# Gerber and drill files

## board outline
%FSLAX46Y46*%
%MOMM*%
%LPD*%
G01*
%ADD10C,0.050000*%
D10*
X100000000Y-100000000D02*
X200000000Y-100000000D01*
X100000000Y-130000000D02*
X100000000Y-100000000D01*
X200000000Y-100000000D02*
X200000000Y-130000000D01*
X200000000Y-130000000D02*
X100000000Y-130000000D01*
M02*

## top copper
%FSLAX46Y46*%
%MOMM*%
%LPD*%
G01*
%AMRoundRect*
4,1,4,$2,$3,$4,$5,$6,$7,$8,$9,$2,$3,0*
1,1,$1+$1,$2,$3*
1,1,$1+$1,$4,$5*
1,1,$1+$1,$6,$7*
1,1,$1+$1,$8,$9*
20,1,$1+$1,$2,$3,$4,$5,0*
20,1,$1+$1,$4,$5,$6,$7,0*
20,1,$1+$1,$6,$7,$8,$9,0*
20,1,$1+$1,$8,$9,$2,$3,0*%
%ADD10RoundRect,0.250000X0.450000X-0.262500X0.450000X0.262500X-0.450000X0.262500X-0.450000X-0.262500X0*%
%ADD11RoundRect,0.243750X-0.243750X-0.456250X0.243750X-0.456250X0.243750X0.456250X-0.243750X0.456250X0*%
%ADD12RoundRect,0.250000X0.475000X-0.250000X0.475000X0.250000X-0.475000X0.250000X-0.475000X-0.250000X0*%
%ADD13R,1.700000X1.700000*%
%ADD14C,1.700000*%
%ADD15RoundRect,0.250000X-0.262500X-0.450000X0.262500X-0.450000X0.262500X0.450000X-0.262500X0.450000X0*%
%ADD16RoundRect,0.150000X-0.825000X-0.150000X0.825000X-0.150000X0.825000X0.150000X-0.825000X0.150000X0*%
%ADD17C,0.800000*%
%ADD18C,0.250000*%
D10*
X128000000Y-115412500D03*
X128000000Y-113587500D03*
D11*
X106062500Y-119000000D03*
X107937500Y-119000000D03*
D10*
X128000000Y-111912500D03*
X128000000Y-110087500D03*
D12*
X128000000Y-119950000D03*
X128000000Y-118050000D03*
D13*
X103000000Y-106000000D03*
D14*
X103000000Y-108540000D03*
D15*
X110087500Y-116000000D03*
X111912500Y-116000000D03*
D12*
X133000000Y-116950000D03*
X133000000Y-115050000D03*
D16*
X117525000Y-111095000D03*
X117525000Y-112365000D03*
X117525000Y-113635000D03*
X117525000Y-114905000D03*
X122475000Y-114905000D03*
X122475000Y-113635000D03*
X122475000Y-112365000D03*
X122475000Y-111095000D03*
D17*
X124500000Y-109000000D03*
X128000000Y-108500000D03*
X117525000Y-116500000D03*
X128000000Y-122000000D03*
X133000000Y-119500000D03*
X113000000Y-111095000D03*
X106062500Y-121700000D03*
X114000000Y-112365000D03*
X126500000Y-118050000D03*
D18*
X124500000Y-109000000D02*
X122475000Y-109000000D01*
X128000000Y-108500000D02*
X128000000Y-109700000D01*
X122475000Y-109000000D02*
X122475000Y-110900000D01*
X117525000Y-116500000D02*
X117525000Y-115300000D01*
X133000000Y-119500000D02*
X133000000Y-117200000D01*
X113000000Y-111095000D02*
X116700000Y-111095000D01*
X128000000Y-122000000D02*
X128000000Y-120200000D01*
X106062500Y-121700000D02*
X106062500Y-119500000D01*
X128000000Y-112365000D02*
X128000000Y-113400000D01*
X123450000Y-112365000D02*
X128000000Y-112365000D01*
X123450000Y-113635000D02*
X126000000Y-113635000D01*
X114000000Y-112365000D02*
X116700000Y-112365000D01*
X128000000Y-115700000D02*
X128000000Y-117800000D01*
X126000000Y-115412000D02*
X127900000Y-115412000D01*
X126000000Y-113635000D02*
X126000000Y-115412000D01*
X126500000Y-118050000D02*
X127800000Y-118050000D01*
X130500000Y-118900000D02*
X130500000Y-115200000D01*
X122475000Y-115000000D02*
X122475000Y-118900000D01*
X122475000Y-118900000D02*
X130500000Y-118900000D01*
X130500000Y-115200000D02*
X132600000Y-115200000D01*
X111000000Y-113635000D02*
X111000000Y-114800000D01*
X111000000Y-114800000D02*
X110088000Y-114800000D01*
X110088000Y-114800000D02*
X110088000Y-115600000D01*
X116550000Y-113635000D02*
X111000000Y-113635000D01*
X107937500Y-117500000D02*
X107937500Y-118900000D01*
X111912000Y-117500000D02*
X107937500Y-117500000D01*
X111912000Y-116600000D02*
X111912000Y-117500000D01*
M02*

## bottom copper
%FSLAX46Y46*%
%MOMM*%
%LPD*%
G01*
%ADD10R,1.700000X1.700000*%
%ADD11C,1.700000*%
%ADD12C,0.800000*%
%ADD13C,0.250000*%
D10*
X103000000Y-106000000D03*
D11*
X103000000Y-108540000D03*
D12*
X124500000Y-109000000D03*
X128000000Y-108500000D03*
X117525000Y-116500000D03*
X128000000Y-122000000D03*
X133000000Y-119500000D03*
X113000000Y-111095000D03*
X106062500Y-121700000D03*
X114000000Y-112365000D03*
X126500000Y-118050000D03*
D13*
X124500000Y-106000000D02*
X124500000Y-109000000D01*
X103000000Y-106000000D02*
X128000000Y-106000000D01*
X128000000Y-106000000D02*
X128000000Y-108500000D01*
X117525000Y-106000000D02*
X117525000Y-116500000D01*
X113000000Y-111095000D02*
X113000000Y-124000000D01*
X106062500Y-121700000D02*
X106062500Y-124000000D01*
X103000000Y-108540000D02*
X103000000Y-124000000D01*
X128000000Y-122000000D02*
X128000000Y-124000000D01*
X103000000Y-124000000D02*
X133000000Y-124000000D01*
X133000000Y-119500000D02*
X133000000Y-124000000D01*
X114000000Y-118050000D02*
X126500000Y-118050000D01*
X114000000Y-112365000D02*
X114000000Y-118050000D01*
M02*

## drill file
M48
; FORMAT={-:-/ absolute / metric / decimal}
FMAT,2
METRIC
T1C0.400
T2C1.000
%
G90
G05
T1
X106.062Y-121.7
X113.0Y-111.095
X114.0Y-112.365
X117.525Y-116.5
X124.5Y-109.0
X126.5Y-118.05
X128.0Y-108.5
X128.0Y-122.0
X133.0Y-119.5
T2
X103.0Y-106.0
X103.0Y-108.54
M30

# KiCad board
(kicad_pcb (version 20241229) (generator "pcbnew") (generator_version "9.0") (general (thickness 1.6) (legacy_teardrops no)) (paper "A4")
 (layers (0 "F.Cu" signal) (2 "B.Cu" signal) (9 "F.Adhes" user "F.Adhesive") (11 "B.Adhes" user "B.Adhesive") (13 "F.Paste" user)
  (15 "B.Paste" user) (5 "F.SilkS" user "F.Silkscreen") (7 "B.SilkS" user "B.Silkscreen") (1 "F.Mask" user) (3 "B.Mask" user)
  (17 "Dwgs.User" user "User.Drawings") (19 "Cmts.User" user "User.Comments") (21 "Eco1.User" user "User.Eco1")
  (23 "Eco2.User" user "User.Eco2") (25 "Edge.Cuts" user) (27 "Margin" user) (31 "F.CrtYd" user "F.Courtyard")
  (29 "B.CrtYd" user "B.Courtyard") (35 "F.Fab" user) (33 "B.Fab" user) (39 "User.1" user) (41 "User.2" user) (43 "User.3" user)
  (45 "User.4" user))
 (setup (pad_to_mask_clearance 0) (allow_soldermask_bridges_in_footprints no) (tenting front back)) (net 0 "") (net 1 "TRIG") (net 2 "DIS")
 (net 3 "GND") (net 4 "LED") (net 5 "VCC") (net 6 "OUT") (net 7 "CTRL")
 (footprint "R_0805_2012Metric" (layer "F.Cu") (at 128 114.5 90)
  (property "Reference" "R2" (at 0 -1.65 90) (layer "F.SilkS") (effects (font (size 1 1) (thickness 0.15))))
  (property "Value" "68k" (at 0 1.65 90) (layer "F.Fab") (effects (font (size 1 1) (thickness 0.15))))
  (pad "1" smd roundrect (at -0.9125 0 90) (size 1.025 1.4) (layers "F.Cu" "F.Mask" "F.Paste") (roundrect_rratio 0.243902) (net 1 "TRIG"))
  (pad "2" smd roundrect (at 0.9125 0 90) (size 1.025 1.4) (layers "F.Cu" "F.Mask" "F.Paste") (roundrect_rratio 0.243902) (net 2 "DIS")))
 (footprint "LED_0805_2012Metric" (layer "F.Cu") (at 107 119)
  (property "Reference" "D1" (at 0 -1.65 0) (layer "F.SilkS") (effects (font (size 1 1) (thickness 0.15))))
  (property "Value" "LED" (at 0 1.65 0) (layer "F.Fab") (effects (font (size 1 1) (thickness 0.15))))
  (pad "1" smd roundrect (at -0.9375 0) (size 0.975 1.4) (layers "F.Cu" "F.Mask" "F.Paste") (roundrect_rratio 0.25) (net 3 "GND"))
  (pad "2" smd roundrect (at 0.9375 0) (size 0.975 1.4) (layers "F.Cu" "F.Mask" "F.Paste") (roundrect_rratio 0.25) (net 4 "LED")))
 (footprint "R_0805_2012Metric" (layer "F.Cu") (at 128 111 90)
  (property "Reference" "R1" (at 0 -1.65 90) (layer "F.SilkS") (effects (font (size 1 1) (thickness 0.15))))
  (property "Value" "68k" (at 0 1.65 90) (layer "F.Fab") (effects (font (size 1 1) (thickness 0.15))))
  (pad "1" smd roundrect (at -0.9125 0 90) (size 1.025 1.4) (layers "F.Cu" "F.Mask" "F.Paste") (roundrect_rratio 0.243902) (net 2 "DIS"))
  (pad "2" smd roundrect (at 0.9125 0 90) (size 1.025 1.4) (layers "F.Cu" "F.Mask" "F.Paste") (roundrect_rratio 0.243902) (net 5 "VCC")))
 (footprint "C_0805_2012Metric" (layer "F.Cu") (at 128 119 90)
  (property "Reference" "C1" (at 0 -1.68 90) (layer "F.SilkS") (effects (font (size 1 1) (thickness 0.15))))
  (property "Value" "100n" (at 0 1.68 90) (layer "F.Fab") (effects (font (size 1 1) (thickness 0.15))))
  (pad "1" smd roundrect (at -0.95 0 90) (size 1 1.45) (layers "F.Cu" "F.Mask" "F.Paste") (roundrect_rratio 0.25) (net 3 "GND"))
  (pad "2" smd roundrect (at 0.95 0 90) (size 1 1.45) (layers "F.Cu" "F.Mask" "F.Paste") (roundrect_rratio 0.25) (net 1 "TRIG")))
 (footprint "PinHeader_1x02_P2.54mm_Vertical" (layer "F.Cu") (at 103 106)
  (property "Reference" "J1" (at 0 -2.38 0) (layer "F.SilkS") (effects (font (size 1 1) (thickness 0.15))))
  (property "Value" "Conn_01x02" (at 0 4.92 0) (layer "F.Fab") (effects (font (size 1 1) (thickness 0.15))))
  (pad "1" thru_hole rect (at 0 0) (size 1.7 1.7) (drill 1) (layers "*.Cu" "*.Mask") (remove_unused_layers no) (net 5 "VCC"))
  (pad "2" thru_hole circle (at 0 2.54) (size 1.7 1.7) (drill 1) (layers "*.Cu" "*.Mask") (remove_unused_layers no) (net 3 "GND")))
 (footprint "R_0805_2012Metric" (layer "F.Cu") (at 111 116)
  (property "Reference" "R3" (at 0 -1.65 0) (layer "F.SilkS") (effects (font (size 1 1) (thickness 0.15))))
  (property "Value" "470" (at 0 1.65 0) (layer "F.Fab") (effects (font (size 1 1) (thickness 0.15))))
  (pad "1" smd roundrect (at -0.9125 0) (size 1.025 1.4) (layers "F.Cu" "F.Mask" "F.Paste") (roundrect_rratio 0.243902) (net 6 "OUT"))
  (pad "2" smd roundrect (at 0.9125 0) (size 1.025 1.4) (layers "F.Cu" "F.Mask" "F.Paste") (roundrect_rratio 0.243902) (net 4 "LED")))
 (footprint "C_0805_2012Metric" (layer "F.Cu") (at 133 116 90)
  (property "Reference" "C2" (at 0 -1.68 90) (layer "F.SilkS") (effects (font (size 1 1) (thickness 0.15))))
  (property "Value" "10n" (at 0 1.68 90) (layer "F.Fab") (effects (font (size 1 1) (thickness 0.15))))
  (pad "1" smd roundrect (at -0.95 0 90) (size 1 1.45) (layers "F.Cu" "F.Mask" "F.Paste") (roundrect_rratio 0.25) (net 3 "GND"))
  (pad "2" smd roundrect (at 0.95 0 90) (size 1 1.45) (layers "F.Cu" "F.Mask" "F.Paste") (roundrect_rratio 0.25) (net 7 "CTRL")))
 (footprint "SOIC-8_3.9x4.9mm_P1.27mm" (layer "F.Cu") (at 120 113)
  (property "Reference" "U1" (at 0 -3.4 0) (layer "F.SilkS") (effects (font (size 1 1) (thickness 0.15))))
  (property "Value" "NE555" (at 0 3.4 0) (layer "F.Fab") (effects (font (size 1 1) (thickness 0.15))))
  (pad "1" smd roundrect (at -2.475 -1.905) (size 1.95 0.6) (layers "F.Cu" "F.Mask" "F.Paste") (roundrect_rratio 0.25) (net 3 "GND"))
  (pad "2" smd roundrect (at -2.475 -0.635) (size 1.95 0.6) (layers "F.Cu" "F.Mask" "F.Paste") (roundrect_rratio 0.25) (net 1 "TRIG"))
  (pad "3" smd roundrect (at -2.475 0.635) (size 1.95 0.6) (layers "F.Cu" "F.Mask" "F.Paste") (roundrect_rratio 0.25) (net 6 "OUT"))
  (pad "4" smd roundrect (at -2.475 1.905) (size 1.95 0.6) (layers "F.Cu" "F.Mask" "F.Paste") (roundrect_rratio 0.25) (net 5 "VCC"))
  (pad "5" smd roundrect (at 2.475 1.905) (size 1.95 0.6) (layers "F.Cu" "F.Mask" "F.Paste") (roundrect_rratio 0.25) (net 7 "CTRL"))
  (pad "6" smd roundrect (at 2.475 0.635) (size 1.95 0.6) (layers "F.Cu" "F.Mask" "F.Paste") (roundrect_rratio 0.25) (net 1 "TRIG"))
  (pad "7" smd roundrect (at 2.475 -0.635) (size 1.95 0.6) (layers "F.Cu" "F.Mask" "F.Paste") (roundrect_rratio 0.25) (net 2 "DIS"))
  (pad "8" smd roundrect (at 2.475 -1.905) (size 1.95 0.6) (layers "F.Cu" "F.Mask" "F.Paste") (roundrect_rratio 0.25) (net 5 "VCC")))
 (gr_line (start 100 100) (end 200 100) (stroke (width 0.05) (type default)) (layer "Edge.Cuts"))
 (gr_line (start 100 130) (end 100 100) (stroke (width 0.05) (type default)) (layer "Edge.Cuts"))
 (gr_line (start 200 100) (end 200 130) (stroke (width 0.05) (type default)) (layer "Edge.Cuts"))
 (gr_line (start 200 130) (end 100 130) (stroke (width 0.05) (type default)) (layer "Edge.Cuts"))
 (segment (start 124.5 109) (end 122.475 109) (width 0.25) (layer "F.Cu") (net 5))
 (segment (start 128 108.5) (end 128 109.7) (width 0.25) (layer "F.Cu") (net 5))
 (segment (start 122.475 109) (end 122.475 110.9) (width 0.25) (layer "F.Cu") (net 5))
 (segment (start 117.525 116.5) (end 117.525 115.3) (width 0.25) (layer "F.Cu") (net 5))
 (via (at 124.5 109) (size 0.8) (drill 0.4) (layers "F.Cu" "B.Cu") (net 5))
 (via (at 128 108.5) (size 0.8) (drill 0.4) (layers "F.Cu" "B.Cu") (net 5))
 (via (at 117.525 116.5) (size 0.8) (drill 0.4) (layers "F.Cu" "B.Cu") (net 5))
 (segment (start 124.5 106) (end 124.5 109) (width 0.25) (layer "B.Cu") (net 5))
 (segment (start 103 106) (end 128 106) (width 0.25) (layer "B.Cu") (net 5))
 (segment (start 128 106) (end 128 108.5) (width 0.25) (layer "B.Cu") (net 5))
 (segment (start 117.525 106) (end 117.525 116.5) (width 0.25) (layer "B.Cu") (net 5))
 (segment (start 133 119.5) (end 133 117.2) (width 0.25) (layer "F.Cu") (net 3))
 (segment (start 113 111.095) (end 116.7 111.095) (width 0.25) (layer "F.Cu") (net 3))
 (segment (start 128 122) (end 128 120.2) (width 0.25) (layer "F.Cu") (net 3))
 (segment (start 106.0625 121.7) (end 106.0625 119.5) (width 0.25) (layer "F.Cu") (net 3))
 (via (at 128 122) (size 0.8) (drill 0.4) (layers "F.Cu" "B.Cu") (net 3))
 (via (at 133 119.5) (size 0.8) (drill 0.4) (layers "F.Cu" "B.Cu") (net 3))
 (via (at 113 111.095) (size 0.8) (drill 0.4) (layers "F.Cu" "B.Cu") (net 3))
 (via (at 106.0625 121.7) (size 0.8) (drill 0.4) (layers "F.Cu" "B.Cu") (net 3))
 (segment (start 113 111.095) (end 113 124) (width 0.25) (layer "B.Cu") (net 3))
 (segment (start 106.0625 121.7) (end 106.0625 124) (width 0.25) (layer "B.Cu") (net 3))
 (segment (start 103 108.54) (end 103 124) (width 0.25) (layer "B.Cu") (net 3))
 (segment (start 128 122) (end 128 124) (width 0.25) (layer "B.Cu") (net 3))
 (segment (start 103 124) (end 133 124) (width 0.25) (layer "B.Cu") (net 3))
 (segment (start 133 119.5) (end 133 124) (width 0.25) (layer "B.Cu") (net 3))
 (segment (start 128 112.365) (end 128 113.4) (width 0.25) (layer "F.Cu") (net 2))
 (segment (start 123.45 112.365) (end 128 112.365) (width 0.25) (layer "F.Cu") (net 2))
 (segment (start 123.45 113.635) (end 126 113.635) (width 0.25) (layer "F.Cu") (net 1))
 (segment (start 114 112.365) (end 116.7 112.365) (width 0.25) (layer "F.Cu") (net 1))
 (segment (start 128 115.7) (end 128 117.8) (width 0.25) (layer "F.Cu") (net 1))
 (segment (start 126 115.412) (end 127.9 115.412) (width 0.25) (layer "F.Cu") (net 1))
 (segment (start 126 113.635) (end 126 115.412) (width 0.25) (layer "F.Cu") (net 1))
 (segment (start 126.5 118.05) (end 127.8 118.05) (width 0.25) (layer "F.Cu") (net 1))
 (via (at 114 112.365) (size 0.8) (drill 0.4) (layers "F.Cu" "B.Cu") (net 1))
 (via (at 126.5 118.05) (size 0.8) (drill 0.4) (layers "F.Cu" "B.Cu") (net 1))
 (segment (start 114 118.05) (end 126.5 118.05) (width 0.25) (layer "B.Cu") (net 1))
 (segment (start 114 112.365) (end 114 118.05) (width 0.25) (layer "B.Cu") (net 1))
 (segment (start 130.5 118.9) (end 130.5 115.2) (width 0.25) (layer "F.Cu") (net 7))
 (segment (start 122.475 115) (end 122.475 118.9) (width 0.25) (layer "F.Cu") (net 7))
 (segment (start 122.475 118.9) (end 130.5 118.9) (width 0.25) (layer "F.Cu") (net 7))
 (segment (start 130.5 115.2) (end 132.6 115.2) (width 0.25) (layer "F.Cu") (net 7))
 (segment (start 111 113.635) (end 111 114.8) (width 0.25) (layer "F.Cu") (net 6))
 (segment (start 111 114.8) (end 110.088 114.8) (width 0.25) (layer "F.Cu") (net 6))
 (segment (start 110.088 114.8) (end 110.088 115.6) (width 0.25) (layer "F.Cu") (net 6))
 (segment (start 116.55 113.635) (end 111 113.635) (width 0.25) (layer "F.Cu") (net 6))
 (segment (start 107.9375 117.5) (end 107.9375 118.9) (width 0.25) (layer "F.Cu") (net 4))
 (segment (start 111.912 117.5) (end 107.9375 117.5) (width 0.25) (layer "F.Cu") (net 4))
 (segment (start 111.912 116.6) (end 111.912 117.5) (width 0.25) (layer "F.Cu") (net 4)))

